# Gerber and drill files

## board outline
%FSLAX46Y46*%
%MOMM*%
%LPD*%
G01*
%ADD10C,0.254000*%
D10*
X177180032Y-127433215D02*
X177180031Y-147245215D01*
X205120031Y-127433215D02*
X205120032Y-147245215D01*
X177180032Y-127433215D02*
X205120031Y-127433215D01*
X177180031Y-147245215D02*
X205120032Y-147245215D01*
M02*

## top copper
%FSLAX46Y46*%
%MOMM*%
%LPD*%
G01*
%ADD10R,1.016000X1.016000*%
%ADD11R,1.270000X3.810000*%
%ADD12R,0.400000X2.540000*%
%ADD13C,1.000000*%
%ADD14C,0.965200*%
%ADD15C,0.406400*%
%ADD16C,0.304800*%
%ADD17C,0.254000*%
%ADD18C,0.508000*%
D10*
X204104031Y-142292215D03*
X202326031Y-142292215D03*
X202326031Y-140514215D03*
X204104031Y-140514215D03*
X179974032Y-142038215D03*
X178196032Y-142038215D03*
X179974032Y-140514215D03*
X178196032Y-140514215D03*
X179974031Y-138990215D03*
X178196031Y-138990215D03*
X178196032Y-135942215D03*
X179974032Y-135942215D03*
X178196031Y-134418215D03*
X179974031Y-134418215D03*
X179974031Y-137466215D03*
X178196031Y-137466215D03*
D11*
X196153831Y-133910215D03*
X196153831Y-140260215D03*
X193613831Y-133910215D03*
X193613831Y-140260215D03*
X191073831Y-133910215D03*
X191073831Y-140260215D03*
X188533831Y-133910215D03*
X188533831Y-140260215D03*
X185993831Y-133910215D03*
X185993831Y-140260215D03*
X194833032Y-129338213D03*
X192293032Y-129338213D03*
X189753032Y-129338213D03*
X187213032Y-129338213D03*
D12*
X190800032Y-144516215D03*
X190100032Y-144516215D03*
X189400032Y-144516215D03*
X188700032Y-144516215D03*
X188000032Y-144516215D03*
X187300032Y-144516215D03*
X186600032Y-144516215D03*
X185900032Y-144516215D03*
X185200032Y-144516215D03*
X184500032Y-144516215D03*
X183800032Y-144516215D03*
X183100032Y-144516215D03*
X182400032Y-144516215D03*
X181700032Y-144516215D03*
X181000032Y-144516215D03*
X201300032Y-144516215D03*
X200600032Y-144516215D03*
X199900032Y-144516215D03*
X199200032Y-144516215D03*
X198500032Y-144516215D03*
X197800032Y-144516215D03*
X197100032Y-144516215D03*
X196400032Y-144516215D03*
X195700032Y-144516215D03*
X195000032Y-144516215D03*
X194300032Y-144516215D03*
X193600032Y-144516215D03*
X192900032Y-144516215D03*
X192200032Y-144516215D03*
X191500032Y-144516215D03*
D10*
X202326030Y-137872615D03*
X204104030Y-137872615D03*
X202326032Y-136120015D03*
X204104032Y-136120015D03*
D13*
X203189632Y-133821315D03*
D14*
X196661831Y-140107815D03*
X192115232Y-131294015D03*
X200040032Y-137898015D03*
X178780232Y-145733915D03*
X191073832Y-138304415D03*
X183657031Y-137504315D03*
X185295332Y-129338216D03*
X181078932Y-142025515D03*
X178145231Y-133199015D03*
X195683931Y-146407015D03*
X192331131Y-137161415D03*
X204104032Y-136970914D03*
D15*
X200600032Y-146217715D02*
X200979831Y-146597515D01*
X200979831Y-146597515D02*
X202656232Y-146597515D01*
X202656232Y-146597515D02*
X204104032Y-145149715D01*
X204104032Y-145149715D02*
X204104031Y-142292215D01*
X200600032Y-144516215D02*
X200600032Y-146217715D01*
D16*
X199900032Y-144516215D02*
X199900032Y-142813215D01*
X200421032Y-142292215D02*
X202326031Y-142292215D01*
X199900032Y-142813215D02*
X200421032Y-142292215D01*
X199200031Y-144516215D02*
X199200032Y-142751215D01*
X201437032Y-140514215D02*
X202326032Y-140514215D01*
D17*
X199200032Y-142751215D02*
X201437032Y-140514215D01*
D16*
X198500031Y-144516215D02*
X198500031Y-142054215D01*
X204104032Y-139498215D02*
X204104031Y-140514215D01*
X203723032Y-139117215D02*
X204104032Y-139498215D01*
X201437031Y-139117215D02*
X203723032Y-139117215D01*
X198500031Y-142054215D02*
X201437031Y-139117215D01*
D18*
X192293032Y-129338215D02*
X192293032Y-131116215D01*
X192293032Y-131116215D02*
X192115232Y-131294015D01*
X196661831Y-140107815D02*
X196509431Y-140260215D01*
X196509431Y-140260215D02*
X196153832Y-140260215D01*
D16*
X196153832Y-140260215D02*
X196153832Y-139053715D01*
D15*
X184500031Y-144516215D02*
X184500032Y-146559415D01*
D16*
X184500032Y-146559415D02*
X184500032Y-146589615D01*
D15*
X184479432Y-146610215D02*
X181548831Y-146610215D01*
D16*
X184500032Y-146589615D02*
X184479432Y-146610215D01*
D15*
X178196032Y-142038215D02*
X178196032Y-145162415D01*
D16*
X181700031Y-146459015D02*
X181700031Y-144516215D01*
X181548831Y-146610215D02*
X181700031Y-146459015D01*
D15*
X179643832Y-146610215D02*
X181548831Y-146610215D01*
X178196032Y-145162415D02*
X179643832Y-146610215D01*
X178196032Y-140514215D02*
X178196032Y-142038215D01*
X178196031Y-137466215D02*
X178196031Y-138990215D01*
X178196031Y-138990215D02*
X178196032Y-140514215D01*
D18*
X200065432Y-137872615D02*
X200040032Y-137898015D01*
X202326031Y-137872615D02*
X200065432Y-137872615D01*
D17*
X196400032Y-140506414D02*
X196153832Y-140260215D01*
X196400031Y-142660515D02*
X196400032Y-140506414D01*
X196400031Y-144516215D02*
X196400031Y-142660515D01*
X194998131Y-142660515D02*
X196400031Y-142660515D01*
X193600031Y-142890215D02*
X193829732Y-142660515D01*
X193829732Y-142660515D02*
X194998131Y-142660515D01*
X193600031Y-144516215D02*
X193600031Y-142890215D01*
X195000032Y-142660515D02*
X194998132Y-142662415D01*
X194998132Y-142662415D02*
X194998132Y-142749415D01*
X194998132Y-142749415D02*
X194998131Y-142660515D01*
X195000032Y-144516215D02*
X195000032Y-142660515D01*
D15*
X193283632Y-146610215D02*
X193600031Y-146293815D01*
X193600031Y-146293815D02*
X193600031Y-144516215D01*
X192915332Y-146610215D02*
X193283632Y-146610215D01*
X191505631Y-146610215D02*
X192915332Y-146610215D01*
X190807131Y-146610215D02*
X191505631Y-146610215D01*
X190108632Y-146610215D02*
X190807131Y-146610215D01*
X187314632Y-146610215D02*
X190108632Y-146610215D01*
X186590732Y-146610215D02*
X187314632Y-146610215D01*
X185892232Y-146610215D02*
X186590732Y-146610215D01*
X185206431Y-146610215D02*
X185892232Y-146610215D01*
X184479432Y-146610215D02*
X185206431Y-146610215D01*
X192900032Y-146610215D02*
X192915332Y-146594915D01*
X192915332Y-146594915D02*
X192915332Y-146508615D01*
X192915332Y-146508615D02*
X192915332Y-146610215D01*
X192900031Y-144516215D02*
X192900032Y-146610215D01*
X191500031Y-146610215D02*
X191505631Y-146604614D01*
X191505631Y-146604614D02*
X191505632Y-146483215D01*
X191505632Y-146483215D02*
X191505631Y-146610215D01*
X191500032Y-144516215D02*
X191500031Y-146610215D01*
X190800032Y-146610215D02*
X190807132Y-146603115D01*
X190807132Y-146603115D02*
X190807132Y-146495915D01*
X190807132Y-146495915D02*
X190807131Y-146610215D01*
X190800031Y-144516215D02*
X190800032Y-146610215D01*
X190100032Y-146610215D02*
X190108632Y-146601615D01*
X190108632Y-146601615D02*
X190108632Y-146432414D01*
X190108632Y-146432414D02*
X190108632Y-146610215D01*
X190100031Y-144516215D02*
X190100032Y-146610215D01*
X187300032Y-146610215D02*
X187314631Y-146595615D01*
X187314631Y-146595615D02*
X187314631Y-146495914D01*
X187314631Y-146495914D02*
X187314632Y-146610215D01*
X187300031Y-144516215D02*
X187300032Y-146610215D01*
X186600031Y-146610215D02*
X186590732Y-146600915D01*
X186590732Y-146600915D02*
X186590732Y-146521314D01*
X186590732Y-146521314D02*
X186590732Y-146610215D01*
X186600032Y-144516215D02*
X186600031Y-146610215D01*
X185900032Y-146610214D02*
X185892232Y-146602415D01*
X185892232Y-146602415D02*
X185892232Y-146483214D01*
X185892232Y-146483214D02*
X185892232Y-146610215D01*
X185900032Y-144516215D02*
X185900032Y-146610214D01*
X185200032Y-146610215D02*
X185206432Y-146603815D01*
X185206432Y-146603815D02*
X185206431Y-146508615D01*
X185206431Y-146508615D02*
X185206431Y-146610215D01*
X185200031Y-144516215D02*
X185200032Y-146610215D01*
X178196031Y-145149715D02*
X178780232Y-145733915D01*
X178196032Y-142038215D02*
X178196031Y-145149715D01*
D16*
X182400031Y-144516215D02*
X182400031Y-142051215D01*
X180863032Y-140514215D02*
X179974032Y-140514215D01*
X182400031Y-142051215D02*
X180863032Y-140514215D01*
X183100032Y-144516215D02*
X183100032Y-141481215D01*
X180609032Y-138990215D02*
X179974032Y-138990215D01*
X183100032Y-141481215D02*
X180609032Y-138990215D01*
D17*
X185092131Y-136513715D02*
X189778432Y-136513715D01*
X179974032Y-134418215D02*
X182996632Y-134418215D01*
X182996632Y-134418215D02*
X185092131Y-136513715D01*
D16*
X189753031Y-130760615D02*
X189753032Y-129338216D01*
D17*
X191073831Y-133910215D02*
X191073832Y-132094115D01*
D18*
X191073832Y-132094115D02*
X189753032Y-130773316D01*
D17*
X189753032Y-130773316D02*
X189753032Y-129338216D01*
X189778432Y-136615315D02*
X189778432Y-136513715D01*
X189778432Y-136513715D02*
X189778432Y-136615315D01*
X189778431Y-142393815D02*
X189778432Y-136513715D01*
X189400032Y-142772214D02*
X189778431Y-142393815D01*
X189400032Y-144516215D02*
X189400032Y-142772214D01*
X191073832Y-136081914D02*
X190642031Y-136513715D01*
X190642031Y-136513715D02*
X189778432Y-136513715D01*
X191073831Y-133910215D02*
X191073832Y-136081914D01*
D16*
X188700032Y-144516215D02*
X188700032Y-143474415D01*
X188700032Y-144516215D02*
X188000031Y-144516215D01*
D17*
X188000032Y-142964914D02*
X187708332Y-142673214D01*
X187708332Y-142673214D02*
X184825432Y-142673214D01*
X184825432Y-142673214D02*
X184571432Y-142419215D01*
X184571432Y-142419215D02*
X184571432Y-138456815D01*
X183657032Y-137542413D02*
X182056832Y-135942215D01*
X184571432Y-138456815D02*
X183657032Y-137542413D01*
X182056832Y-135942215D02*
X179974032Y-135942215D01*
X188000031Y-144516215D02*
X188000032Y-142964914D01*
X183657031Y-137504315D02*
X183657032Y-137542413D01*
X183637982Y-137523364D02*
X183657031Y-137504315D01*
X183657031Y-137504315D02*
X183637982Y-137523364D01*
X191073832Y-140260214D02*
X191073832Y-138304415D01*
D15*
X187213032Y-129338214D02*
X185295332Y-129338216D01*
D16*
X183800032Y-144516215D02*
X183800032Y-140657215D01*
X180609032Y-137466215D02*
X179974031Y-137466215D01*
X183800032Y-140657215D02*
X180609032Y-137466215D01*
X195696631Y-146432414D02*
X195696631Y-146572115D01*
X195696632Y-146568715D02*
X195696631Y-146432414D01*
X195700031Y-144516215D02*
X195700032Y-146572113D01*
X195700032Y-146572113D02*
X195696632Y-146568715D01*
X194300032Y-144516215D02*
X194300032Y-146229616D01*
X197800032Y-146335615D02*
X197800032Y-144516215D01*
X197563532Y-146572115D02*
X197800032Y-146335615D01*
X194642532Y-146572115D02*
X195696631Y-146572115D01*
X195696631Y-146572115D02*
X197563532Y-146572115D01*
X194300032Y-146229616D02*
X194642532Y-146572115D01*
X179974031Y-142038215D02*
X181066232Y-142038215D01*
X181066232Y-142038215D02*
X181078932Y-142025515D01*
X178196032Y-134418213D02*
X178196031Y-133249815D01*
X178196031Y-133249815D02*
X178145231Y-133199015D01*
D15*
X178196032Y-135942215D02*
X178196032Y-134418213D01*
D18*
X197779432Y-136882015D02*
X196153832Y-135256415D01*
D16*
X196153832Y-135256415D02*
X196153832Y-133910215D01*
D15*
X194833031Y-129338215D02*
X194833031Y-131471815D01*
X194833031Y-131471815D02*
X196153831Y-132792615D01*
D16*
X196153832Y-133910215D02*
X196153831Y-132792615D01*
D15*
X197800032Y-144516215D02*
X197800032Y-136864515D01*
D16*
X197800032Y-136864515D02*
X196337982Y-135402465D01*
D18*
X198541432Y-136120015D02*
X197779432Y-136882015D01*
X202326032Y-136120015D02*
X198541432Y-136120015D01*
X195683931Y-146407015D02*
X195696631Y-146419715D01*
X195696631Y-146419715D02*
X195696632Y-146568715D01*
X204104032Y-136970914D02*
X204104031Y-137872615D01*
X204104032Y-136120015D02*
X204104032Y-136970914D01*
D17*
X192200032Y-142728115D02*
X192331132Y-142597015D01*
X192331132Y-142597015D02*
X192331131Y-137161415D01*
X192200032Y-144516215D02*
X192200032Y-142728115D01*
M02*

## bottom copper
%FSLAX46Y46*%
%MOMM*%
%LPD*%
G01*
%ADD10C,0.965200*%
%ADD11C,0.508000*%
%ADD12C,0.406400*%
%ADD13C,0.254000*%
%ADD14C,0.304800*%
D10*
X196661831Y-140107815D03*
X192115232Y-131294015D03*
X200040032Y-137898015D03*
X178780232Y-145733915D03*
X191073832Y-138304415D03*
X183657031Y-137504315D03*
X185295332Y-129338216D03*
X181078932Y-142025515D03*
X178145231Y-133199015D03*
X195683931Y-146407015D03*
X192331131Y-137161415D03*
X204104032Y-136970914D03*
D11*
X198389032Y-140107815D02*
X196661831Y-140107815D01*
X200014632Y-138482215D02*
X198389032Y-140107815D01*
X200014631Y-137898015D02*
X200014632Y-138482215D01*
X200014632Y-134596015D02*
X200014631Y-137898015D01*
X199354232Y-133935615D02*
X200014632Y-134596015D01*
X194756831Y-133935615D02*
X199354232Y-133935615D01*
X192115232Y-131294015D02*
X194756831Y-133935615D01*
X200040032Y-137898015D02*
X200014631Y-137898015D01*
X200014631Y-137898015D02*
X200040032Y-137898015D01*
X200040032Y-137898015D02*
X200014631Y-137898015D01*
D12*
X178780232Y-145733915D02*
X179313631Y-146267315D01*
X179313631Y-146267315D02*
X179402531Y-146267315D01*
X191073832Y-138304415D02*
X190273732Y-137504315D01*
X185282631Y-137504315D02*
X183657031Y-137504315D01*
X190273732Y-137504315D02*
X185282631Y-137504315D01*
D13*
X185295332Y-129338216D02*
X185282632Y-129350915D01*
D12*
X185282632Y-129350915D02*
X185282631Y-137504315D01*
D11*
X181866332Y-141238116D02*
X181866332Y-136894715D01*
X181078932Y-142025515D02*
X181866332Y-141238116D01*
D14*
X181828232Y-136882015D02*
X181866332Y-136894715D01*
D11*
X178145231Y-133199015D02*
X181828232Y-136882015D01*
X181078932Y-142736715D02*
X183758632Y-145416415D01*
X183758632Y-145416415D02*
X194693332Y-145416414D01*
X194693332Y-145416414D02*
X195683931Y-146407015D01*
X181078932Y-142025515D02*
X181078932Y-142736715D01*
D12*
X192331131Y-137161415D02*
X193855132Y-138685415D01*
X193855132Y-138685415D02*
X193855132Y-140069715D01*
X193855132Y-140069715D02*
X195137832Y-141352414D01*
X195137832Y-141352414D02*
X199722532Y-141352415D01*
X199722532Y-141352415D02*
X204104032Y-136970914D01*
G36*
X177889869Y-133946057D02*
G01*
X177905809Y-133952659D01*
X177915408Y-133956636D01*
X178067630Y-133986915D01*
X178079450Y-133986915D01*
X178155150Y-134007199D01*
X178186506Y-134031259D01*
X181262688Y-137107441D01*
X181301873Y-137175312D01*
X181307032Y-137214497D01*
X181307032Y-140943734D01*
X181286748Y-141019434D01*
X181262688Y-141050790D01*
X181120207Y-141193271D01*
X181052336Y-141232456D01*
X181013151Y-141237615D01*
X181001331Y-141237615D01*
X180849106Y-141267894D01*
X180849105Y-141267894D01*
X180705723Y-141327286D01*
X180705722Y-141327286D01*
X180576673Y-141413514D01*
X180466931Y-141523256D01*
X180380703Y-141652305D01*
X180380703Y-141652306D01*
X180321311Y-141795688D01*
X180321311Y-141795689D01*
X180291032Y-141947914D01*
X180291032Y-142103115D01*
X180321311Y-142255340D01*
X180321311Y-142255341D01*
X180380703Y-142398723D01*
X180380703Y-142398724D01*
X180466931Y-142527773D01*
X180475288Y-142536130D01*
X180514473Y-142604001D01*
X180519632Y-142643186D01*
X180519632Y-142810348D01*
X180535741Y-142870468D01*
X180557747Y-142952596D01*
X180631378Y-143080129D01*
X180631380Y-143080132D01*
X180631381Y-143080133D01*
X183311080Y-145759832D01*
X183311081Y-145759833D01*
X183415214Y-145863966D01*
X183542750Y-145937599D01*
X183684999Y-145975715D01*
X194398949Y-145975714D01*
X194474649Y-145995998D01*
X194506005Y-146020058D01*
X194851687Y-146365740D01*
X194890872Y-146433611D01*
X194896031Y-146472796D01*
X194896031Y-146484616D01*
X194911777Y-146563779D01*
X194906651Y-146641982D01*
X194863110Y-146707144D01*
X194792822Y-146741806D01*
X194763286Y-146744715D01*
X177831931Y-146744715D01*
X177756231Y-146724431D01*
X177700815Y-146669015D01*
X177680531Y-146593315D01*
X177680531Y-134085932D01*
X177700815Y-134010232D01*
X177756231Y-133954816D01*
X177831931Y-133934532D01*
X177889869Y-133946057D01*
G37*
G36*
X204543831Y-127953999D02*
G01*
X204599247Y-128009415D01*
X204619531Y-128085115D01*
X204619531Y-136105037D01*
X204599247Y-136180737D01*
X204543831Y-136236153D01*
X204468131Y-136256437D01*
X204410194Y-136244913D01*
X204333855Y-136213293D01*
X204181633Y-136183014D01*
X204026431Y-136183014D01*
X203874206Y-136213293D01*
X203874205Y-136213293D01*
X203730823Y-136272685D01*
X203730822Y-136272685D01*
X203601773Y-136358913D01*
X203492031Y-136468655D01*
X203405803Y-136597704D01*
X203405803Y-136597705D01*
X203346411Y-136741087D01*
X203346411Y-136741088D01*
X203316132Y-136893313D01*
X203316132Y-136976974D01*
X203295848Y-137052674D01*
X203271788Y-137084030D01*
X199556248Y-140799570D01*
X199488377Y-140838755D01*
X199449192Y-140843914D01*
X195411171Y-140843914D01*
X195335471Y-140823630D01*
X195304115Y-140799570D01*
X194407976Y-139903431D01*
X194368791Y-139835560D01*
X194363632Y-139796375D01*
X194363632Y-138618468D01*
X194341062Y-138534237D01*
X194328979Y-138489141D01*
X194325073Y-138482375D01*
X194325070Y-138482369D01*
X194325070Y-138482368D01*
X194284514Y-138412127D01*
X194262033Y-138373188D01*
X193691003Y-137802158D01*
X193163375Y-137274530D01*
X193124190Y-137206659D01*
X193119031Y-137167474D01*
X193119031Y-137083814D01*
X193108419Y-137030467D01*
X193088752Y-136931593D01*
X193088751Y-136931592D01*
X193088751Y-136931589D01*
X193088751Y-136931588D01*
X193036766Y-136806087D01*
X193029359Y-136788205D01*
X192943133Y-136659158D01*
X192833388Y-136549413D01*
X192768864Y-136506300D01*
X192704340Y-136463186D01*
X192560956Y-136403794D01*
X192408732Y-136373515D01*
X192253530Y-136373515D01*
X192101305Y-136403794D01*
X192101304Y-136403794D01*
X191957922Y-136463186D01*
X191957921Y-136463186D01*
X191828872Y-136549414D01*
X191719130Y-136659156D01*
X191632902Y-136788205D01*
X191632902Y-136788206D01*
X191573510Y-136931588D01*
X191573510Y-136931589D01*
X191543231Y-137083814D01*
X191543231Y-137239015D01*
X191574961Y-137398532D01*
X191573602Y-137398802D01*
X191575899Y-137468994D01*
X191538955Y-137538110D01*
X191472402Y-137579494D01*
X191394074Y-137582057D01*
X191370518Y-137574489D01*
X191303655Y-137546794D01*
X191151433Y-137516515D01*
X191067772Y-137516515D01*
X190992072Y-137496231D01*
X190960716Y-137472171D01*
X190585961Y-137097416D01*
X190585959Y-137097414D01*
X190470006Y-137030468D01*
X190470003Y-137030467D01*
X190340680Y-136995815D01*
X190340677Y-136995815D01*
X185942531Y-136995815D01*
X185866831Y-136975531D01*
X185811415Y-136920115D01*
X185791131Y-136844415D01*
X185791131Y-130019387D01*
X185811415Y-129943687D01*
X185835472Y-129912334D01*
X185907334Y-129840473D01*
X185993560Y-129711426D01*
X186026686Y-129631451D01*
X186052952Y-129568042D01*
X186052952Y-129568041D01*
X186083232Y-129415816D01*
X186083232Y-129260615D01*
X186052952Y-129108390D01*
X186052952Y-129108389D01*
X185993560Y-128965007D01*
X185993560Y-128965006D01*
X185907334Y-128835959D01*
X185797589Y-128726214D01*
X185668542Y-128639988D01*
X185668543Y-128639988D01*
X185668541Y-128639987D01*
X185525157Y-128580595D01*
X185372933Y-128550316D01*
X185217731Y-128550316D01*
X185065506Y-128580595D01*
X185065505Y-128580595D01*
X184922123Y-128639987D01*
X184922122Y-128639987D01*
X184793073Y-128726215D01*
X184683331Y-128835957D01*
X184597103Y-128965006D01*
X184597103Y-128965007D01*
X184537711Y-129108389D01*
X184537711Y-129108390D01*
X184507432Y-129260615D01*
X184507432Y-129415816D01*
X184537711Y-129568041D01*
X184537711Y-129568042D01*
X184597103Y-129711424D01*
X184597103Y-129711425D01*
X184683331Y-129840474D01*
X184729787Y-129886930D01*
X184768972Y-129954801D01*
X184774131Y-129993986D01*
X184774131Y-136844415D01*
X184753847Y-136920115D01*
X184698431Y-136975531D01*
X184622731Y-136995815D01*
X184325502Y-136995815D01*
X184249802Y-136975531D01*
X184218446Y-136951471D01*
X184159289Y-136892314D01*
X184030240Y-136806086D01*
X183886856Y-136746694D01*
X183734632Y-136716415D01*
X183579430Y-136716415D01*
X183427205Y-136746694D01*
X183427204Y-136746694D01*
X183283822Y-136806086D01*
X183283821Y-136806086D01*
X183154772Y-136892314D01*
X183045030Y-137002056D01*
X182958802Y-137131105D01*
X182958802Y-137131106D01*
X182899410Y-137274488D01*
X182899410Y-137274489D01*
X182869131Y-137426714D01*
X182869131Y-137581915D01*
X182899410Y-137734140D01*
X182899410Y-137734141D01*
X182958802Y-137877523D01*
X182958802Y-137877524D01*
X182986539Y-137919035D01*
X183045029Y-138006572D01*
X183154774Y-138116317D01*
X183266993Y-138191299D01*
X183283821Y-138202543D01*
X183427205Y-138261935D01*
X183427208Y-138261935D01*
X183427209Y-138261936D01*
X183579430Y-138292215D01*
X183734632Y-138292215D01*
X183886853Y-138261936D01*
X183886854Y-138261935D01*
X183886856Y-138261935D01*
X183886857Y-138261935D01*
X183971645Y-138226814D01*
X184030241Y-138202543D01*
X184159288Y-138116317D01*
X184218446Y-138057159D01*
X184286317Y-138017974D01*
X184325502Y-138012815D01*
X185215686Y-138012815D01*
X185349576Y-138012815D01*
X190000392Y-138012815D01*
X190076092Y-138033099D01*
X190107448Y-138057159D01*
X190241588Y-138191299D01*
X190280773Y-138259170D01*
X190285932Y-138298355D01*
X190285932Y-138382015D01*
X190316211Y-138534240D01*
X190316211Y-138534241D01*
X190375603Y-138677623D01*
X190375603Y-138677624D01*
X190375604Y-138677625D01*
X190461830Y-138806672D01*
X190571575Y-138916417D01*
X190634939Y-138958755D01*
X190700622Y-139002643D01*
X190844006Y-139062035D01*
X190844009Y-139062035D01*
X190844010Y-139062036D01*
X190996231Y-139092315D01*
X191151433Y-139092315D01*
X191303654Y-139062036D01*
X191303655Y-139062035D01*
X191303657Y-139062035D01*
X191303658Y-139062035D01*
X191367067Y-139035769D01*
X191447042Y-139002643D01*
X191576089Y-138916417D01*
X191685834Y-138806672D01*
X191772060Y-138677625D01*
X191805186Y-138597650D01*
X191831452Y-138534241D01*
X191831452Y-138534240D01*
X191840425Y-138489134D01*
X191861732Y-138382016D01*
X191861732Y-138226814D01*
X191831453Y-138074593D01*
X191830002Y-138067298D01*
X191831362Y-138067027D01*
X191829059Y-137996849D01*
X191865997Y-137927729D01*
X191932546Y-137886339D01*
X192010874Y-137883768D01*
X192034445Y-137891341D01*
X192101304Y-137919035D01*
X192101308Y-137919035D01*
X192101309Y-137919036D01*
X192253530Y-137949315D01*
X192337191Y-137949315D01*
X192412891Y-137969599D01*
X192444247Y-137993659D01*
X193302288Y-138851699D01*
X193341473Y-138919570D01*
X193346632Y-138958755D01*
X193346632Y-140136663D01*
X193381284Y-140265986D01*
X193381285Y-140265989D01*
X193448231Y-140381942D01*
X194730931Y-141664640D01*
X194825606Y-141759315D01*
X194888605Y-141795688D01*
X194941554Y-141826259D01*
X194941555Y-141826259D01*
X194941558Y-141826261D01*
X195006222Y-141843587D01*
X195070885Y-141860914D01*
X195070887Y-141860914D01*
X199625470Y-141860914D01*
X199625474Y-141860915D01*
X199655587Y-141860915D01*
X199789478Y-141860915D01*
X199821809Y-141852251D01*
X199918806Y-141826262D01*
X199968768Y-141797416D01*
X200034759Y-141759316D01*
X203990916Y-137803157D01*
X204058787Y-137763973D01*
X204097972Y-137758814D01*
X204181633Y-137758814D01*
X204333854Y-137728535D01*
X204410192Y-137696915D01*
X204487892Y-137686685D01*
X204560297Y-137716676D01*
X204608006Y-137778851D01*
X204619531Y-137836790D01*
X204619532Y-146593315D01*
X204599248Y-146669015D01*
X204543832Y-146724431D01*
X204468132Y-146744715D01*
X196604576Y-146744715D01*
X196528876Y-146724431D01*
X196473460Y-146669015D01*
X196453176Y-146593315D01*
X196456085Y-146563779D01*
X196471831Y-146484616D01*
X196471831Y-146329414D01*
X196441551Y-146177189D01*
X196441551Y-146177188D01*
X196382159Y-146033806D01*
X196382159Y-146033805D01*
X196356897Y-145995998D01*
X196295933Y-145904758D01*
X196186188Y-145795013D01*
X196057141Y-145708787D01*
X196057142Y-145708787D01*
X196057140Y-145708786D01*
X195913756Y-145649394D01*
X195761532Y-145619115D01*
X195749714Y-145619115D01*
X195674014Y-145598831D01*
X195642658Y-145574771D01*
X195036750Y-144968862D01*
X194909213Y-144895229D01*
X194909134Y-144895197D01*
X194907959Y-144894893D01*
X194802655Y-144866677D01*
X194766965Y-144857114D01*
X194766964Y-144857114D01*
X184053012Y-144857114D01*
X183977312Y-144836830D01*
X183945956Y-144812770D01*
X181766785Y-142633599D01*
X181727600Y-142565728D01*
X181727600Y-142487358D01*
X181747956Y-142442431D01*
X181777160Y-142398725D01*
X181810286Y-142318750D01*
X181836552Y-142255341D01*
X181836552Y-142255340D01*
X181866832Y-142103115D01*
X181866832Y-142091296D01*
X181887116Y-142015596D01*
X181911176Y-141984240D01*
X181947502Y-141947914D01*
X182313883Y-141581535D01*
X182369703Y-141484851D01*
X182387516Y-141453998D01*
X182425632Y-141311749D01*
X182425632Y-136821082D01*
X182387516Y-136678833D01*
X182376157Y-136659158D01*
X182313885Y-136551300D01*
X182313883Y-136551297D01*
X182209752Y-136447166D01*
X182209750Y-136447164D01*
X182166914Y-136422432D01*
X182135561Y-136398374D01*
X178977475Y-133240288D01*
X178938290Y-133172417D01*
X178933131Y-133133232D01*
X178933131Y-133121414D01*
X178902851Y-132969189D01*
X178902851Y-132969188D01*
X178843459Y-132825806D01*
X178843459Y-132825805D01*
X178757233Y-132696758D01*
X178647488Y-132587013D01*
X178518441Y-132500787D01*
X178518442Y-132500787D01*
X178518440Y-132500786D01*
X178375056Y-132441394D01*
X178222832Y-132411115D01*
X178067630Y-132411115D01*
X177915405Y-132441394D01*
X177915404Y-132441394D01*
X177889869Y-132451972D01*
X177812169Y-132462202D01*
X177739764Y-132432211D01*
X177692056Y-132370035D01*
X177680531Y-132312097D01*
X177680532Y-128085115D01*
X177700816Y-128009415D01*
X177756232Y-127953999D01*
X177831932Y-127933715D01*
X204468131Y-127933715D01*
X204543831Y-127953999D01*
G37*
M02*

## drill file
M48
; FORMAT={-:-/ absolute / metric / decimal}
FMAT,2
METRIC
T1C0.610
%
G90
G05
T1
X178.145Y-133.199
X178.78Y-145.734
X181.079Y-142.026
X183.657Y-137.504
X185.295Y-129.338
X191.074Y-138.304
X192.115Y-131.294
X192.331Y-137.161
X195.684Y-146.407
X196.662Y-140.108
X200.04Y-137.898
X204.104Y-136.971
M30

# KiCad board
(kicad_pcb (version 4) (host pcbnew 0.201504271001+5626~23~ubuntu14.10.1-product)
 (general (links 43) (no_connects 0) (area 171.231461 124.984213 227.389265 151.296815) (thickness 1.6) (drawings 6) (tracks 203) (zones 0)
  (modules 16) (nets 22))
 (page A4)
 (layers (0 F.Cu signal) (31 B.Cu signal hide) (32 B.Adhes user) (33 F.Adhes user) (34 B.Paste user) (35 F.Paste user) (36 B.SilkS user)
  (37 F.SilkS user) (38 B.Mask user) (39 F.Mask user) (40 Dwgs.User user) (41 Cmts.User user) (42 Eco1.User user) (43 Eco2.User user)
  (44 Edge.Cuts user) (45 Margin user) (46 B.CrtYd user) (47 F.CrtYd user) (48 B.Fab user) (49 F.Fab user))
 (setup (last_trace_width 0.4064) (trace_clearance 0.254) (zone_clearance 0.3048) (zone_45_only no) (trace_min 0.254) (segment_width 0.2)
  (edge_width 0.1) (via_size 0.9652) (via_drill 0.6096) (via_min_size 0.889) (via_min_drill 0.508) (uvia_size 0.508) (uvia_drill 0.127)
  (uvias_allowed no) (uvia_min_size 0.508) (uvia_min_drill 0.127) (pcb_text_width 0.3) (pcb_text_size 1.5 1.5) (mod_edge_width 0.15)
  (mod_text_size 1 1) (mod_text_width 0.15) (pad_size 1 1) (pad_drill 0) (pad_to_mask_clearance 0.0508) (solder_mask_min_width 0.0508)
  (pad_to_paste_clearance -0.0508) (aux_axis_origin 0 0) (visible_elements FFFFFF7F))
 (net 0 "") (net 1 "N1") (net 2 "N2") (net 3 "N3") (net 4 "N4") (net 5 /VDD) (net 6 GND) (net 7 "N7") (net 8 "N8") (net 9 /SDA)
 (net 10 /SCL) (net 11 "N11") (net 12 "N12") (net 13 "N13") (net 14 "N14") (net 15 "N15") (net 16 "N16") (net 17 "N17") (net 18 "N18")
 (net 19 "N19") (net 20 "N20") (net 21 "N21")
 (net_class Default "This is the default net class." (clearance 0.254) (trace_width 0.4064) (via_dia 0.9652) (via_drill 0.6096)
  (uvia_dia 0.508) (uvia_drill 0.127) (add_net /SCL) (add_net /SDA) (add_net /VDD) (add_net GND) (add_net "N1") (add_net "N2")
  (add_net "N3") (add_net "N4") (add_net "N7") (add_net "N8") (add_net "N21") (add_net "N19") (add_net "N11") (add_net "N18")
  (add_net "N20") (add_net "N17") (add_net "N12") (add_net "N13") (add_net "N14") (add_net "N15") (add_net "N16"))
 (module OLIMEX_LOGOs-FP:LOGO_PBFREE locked (layer F.Cu) (at 202.8444 130.2258)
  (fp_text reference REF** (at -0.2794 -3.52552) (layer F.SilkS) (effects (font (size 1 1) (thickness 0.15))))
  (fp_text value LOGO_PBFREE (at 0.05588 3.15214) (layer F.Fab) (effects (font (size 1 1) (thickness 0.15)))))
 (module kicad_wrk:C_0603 (layer F.Cu) (at 203.215031 142.292215 180)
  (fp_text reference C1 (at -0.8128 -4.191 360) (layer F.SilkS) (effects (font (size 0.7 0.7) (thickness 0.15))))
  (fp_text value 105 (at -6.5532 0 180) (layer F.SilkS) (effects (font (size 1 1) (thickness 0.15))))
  (pad 1 smd rect (at -0.889 0 180) (size 1.016 1.016) (layers F.Cu F.Paste F.Mask) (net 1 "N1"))
  (pad 2 smd rect (at 0.889 0 180) (size 1.016 1.016) (layers F.Cu F.Paste F.Mask) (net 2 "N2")))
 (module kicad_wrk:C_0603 (layer F.Cu) (at 203.215031 140.514215)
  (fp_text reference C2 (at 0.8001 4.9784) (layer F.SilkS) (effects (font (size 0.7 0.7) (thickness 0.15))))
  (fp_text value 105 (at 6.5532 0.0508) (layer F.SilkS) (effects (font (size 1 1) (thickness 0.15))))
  (pad 1 smd rect (at -0.889 0) (size 1.016 1.016) (layers F.Cu F.Paste F.Mask) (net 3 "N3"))
  (pad 2 smd rect (at 0.889 0) (size 1.016 1.016) (layers F.Cu F.Paste F.Mask) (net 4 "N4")))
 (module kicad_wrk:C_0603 (layer F.Cu) (at 179.085032 142.038215 180)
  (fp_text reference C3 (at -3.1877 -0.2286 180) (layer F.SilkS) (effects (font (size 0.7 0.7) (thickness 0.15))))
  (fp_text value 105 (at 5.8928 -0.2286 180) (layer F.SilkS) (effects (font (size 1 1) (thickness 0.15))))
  (pad 1 smd rect (at -0.889 0 180) (size 1.016 1.016) (layers F.Cu F.Paste F.Mask) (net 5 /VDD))
  (pad 2 smd rect (at 0.889 0 180) (size 1.016 1.016) (layers F.Cu F.Paste F.Mask) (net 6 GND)))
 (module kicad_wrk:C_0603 (layer F.Cu) (at 179.085032 140.514215 180)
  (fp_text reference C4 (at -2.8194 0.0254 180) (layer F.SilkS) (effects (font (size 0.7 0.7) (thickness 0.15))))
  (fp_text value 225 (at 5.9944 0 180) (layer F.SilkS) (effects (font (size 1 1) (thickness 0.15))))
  (pad 1 smd rect (at -0.889 0 180) (size 1.016 1.016) (layers F.Cu F.Paste F.Mask) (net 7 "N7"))
  (pad 2 smd rect (at 0.889 0 180) (size 1.016 1.016) (layers F.Cu F.Paste F.Mask) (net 6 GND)))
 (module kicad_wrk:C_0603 (layer F.Cu) (at 179.085031 138.990215 180)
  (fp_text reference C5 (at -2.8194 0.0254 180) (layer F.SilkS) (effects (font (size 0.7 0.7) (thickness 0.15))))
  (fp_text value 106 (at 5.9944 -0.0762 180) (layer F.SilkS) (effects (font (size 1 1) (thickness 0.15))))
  (pad 1 smd rect (at -0.889 0 180) (size 1.016 1.016) (layers F.Cu F.Paste F.Mask) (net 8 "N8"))
  (pad 2 smd rect (at 0.889 0 180) (size 1.016 1.016) (layers F.Cu F.Paste F.Mask) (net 6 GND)))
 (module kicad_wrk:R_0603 (layer F.Cu) (at 179.085032 135.942215)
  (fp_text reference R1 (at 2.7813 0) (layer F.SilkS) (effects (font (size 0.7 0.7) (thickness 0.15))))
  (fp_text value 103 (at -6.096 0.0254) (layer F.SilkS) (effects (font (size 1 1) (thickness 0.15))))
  (pad 1 smd rect (at -0.889 0) (size 1.016 1.016) (layers F.Cu F.Paste F.Mask) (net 5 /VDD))
  (pad 2 smd rect (at 0.889 0) (size 1.016 1.016) (layers F.Cu F.Paste F.Mask) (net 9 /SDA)))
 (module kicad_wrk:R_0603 (layer F.Cu) (at 179.085031 134.418215)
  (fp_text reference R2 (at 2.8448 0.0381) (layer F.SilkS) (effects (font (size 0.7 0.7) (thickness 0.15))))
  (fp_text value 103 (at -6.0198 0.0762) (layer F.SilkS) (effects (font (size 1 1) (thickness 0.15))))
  (pad 1 smd rect (at -0.889 0) (size 1.016 1.016) (layers F.Cu F.Paste F.Mask) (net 5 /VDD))
  (pad 2 smd rect (at 0.889 0) (size 1.016 1.016) (layers F.Cu F.Paste F.Mask) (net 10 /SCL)))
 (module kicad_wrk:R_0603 (layer F.Cu) (at 179.085031 137.466215 180)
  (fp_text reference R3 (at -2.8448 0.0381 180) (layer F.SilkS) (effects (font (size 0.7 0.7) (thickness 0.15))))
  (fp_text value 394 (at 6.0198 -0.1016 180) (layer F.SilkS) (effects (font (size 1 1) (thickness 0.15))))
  (pad 1 smd rect (at -0.889 0 180) (size 1.016 1.016) (layers F.Cu F.Paste F.Mask) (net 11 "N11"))
  (pad 2 smd rect (at 0.889 0 180) (size 1.016 1.016) (layers F.Cu F.Paste F.Mask) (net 6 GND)))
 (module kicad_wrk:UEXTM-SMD (layer F.Cu) (at 191.073831 137.085215)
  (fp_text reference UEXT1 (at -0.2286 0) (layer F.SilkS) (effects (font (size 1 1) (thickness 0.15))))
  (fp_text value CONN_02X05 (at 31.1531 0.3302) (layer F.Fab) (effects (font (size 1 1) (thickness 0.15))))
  (pad 1 smd rect (at 5.08 -3.175) (size 1.27 3.81) (layers F.Cu F.Paste F.Mask) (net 5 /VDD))
  (pad 2 smd rect (at 5.08 3.175) (size 1.27 3.81) (layers F.Cu F.Paste F.Mask) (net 6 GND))
  (pad 3 smd rect (at 2.54 -3.175) (size 1.27 3.81) (layers F.Cu F.Paste F.Mask) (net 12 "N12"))
  (pad 4 smd rect (at 2.54 3.175) (size 1.27 3.81) (layers F.Cu F.Paste F.Mask) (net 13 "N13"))
  (pad 5 smd rect (at 0 -3.175) (size 1.27 3.81) (layers F.Cu F.Paste F.Mask) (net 10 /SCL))
  (pad 6 smd rect (at 0 3.175) (size 1.27 3.81) (layers F.Cu F.Paste F.Mask) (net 9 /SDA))
  (pad 7 smd rect (at -2.54 -3.175) (size 1.27 3.81) (layers F.Cu F.Paste F.Mask) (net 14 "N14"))
  (pad 8 smd rect (at -2.54 3.175) (size 1.27 3.81) (layers F.Cu F.Paste F.Mask) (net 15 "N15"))
  (pad 9 smd rect (at -5.08 -3.175) (size 1.27 3.81) (layers F.Cu F.Paste F.Mask) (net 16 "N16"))
  (pad 10 smd rect (at -5.08 3.175) (size 1.27 3.81) (layers F.Cu F.Paste F.Mask) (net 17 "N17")))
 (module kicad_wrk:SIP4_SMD (layer F.Cu) (at 191.023032 129.338213 180)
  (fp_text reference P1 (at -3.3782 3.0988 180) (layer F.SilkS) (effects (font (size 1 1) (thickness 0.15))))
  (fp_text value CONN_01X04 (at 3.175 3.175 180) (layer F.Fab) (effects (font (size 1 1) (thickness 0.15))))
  (pad 1 smd rect (at -3.81 0 180) (size 1.27 3.81) (layers F.Cu F.Mask) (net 5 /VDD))
  (pad 2 smd rect (at -1.27 0 180) (size 1.27 3.81) (layers F.Cu F.Mask) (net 6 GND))
  (pad 3 smd rect (at 1.27 0 180) (size 1.27 3.81) (layers F.Cu F.Mask) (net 10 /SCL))
  (pad 4 smd rect (at 3.81 0 180) (size 1.27 3.81) (layers F.Cu F.Mask) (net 9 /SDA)))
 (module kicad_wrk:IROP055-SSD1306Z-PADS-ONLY (layer F.Cu) (at 191.150032 143.816215 180)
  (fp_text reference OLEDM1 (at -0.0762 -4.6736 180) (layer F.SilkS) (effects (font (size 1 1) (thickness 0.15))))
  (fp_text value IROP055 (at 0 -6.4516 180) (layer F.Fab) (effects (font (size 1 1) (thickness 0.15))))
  (pad 16 smd rect (at 0.35 -0.7 180) (size 0.4 2.54) (layers F.Cu F.Paste F.Mask) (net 6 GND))
  (pad 17 smd rect (at 1.05 -0.7 180) (size 0.4 2.54) (layers F.Cu F.Paste F.Mask) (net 6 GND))
  (pad 18 smd rect (at 1.75 -0.7 180) (size 0.4 2.54) (layers F.Cu F.Paste F.Mask) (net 10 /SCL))
  (pad 19 smd rect (at 2.45 -0.7 180) (size 0.4 2.54) (layers F.Cu F.Paste F.Mask) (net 9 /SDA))
  (pad 20 smd rect (at 3.15 -0.7 180) (size 0.4 2.54) (layers F.Cu F.Paste F.Mask) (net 9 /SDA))
  (pad 21 smd rect (at 3.85 -0.7 180) (size 0.4 2.54) (layers F.Cu F.Paste F.Mask) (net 6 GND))
  (pad 22 smd rect (at 4.55 -0.7 180) (size 0.4 2.54) (layers F.Cu F.Paste F.Mask) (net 6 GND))
  (pad 23 smd rect (at 5.25 -0.7 180) (size 0.4 2.54) (layers F.Cu F.Paste F.Mask) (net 6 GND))
  (pad 24 smd rect (at 5.95 -0.7 180) (size 0.4 2.54) (layers F.Cu F.Paste F.Mask) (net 6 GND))
  (pad 25 smd rect (at 6.65 -0.7 180) (size 0.4 2.54) (layers F.Cu F.Paste F.Mask) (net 6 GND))
  (pad 26 smd rect (at 7.35 -0.7 180) (size 0.4 2.54) (layers F.Cu F.Paste F.Mask) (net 11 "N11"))
  (pad 27 smd rect (at 8.05 -0.7 180) (size 0.4 2.54) (layers F.Cu F.Paste F.Mask) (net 8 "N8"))
  (pad 28 smd rect (at 8.75 -0.7 180) (size 0.4 2.54) (layers F.Cu F.Paste F.Mask) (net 7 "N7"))
  (pad 29 smd rect (at 9.45 -0.7 180) (size 0.4 2.54) (layers F.Cu F.Paste F.Mask) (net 6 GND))
  (pad 30 smd rect (at 10.15 -0.7 180) (size 0.4 2.54) (layers F.Cu F.Paste F.Mask) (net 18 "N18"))
  (pad 1 smd rect (at -10.15 -0.7 180) (size 0.4 2.54) (layers F.Cu F.Paste F.Mask) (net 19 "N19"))
  (pad 2 smd rect (at -9.45 -0.7 180) (size 0.4 2.54) (layers F.Cu F.Paste F.Mask) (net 1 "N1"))
  (pad 3 smd rect (at -8.75 -0.7 180) (size 0.4 2.54) (layers F.Cu F.Paste F.Mask) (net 2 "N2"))
  (pad 4 smd rect (at -8.05 -0.7 180) (size 0.4 2.54) (layers F.Cu F.Paste F.Mask) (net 3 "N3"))
  (pad 5 smd rect (at -7.35 -0.7 180) (size 0.4 2.54) (layers F.Cu F.Paste F.Mask) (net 4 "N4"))
  (pad 6 smd rect (at -6.65 -0.7 180) (size 0.4 2.54) (layers F.Cu F.Paste F.Mask) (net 5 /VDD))
  (pad 7 smd rect (at -5.95 -0.7 180) (size 0.4 2.54) (layers F.Cu F.Paste F.Mask) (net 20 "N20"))
  (pad 8 smd rect (at -5.25 -0.7 180) (size 0.4 2.54) (layers F.Cu F.Paste F.Mask) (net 6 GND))
  (pad 9 smd rect (at -4.55 -0.7 180) (size 0.4 2.54) (layers F.Cu F.Paste F.Mask) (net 5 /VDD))
  (pad 10 smd rect (at -3.85 -0.7 180) (size 0.4 2.54) (layers F.Cu F.Paste F.Mask) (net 6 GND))
  (pad 11 smd rect (at -3.15 -0.7 180) (size 0.4 2.54) (layers F.Cu F.Paste F.Mask) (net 5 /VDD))
  (pad 12 smd rect (at -2.45 -0.7 180) (size 0.4 2.54) (layers F.Cu F.Paste F.Mask) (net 6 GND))
  (pad 13 smd rect (at -1.75 -0.7 180) (size 0.4 2.54) (layers F.Cu F.Paste F.Mask) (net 6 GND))
  (pad 14 smd rect (at -1.05 -0.7 180) (size 0.4 2.54) (layers F.Cu F.Paste F.Mask) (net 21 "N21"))
  (pad 15 smd rect (at -0.35 -0.7 180) (size 0.4 2.54) (layers F.Cu F.Paste F.Mask) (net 6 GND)))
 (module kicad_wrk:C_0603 (layer F.Cu) (at 203.21503 137.872615)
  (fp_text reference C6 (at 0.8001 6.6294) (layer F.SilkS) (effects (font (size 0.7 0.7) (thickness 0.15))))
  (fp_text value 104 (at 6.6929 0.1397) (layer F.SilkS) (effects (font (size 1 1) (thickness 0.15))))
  (pad 1 smd rect (at -0.889 0) (size 1.016 1.016) (layers F.Cu F.Paste F.Mask) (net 6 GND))
  (pad 2 smd rect (at 0.889 0) (size 1.016 1.016) (layers F.Cu F.Paste F.Mask) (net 21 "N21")))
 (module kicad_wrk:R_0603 (layer F.Cu) (at 203.215032 136.120015)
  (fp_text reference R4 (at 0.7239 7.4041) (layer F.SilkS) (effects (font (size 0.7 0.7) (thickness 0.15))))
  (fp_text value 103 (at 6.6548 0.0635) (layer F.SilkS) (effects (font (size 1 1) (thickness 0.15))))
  (pad 1 smd rect (at -0.889 0) (size 1.016 1.016) (layers F.Cu F.Paste F.Mask) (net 5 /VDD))
  (pad 2 smd rect (at 0.889 0) (size 1.016 1.016) (layers F.Cu F.Paste F.Mask) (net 21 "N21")))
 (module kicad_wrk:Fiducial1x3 (layer F.Cu) (at 203.189632 133.821315 180)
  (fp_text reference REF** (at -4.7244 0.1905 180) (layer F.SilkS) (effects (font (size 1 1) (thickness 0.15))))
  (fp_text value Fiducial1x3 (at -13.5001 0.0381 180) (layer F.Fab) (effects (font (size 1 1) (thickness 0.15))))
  (pad Fid1 smd circle (at 0 0 180) (size 1 1) (layers F.Cu F.Mask)))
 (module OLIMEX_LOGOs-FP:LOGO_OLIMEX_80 (layer F.Cu) (at 180.837632 128.728615)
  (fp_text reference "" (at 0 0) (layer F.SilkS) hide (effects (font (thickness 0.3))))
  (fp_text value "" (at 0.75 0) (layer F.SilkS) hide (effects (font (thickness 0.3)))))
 (gr_line (start 177.180032 127.433215) (end 177.180031 147.245215) (angle 90) (layer Edge.Cuts) (width 0.254))
 (gr_line (start 205.120031 127.433215) (end 205.120032 147.245215) (angle 90) (layer Edge.Cuts) (width 0.254))
 (gr_line (start 177.180032 127.433215) (end 205.120031 127.433215) (angle 90) (layer Edge.Cuts) (width 0.254))
 (gr_line (start 177.180031 147.245215) (end 205.120032 147.245215) (angle 90) (layer Edge.Cuts) (width 0.254))
 (segment (start 200.600032 146.217715) (end 200.979831 146.597515) (width 0.4064) (layer F.Cu) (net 1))
 (segment (start 200.979831 146.597515) (end 202.656232 146.597515) (width 0.4064) (layer F.Cu) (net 1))
 (segment (start 202.656232 146.597515) (end 204.104032 145.149715) (width 0.4064) (layer F.Cu) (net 1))
 (segment (start 204.104032 145.149715) (end 204.104031 142.292215) (width 0.4064) (layer F.Cu) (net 1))
 (segment (start 200.600032 144.516215) (end 200.600032 146.217715) (width 0.4064) (layer F.Cu) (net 1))
 (segment (start 199.900032 144.516215) (end 199.900032 142.813215) (width 0.3048) (layer F.Cu) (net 2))
 (segment (start 200.421032 142.292215) (end 202.326031 142.292215) (width 0.3048) (layer F.Cu) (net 2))
 (segment (start 199.900032 142.813215) (end 200.421032 142.292215) (width 0.3048) (layer F.Cu) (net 2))
 (segment (start 199.200031 144.516215) (end 199.200032 142.751215) (width 0.3048) (layer F.Cu) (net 3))
 (segment (start 201.437032 140.514215) (end 202.326032 140.514215) (width 0.3048) (layer F.Cu) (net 3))
 (segment (start 199.200032 142.751215) (end 201.437032 140.514215) (width 0.254) (layer F.Cu) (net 3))
 (segment (start 198.500031 144.516215) (end 198.500031 142.054215) (width 0.3048) (layer F.Cu) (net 4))
 (segment (start 204.104032 139.498215) (end 204.104031 140.514215) (width 0.3048) (layer F.Cu) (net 4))
 (segment (start 203.723032 139.117215) (end 204.104032 139.498215) (width 0.3048) (layer F.Cu) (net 4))
 (segment (start 201.437031 139.117215) (end 203.723032 139.117215) (width 0.3048) (layer F.Cu) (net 4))
 (segment (start 198.500031 142.054215) (end 201.437031 139.117215) (width 0.3048) (layer F.Cu) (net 4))
 (segment (start 198.389032 140.107815) (end 196.661831 140.107815) (width 0.508) (layer B.Cu) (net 6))
 (segment (start 200.014632 138.482215) (end 198.389032 140.107815) (width 0.508) (layer B.Cu) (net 6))
 (segment (start 200.014631 137.898015) (end 200.014632 138.482215) (width 0.508) (layer B.Cu) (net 6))
 (segment (start 200.014632 134.596015) (end 200.014631 137.898015) (width 0.508) (layer B.Cu) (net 6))
 (segment (start 199.354232 133.935615) (end 200.014632 134.596015) (width 0.508) (layer B.Cu) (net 6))
 (segment (start 194.756831 133.935615) (end 199.354232 133.935615) (width 0.508) (layer B.Cu) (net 6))
 (segment (start 192.115232 131.294015) (end 194.756831 133.935615) (width 0.508) (layer B.Cu) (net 6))
 (segment (start 192.293032 129.338215) (end 192.293032 131.116215) (width 0.508) (layer F.Cu) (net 6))
 (segment (start 192.293032 131.116215) (end 192.115232 131.294015) (width 0.508) (layer F.Cu) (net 6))
 (segment (start 196.661831 140.107815) (end 196.509431 140.260215) (width 0.508) (layer F.Cu) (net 6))
 (via (at 196.661831 140.107815) (size 0.9652) (layers F.Cu B.Cu) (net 6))
 (via (at 192.115232 131.294015) (size 0.9652) (layers F.Cu B.Cu) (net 6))
 (segment (start 196.509431 140.260215) (end 196.153832 140.260215) (width 0.508) (layer F.Cu) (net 6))
 (segment (start 196.153832 140.260215) (end 196.153832 139.053715) (width 0.3048) (layer F.Cu) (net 6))
 (segment (start 184.500031 144.516215) (end 184.500032 146.559415) (width 0.4064) (layer F.Cu) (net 6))
 (segment (start 184.500032 146.559415) (end 184.500032 146.589615) (width 0.3048) (layer F.Cu) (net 6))
 (segment (start 184.479432 146.610215) (end 181.548831 146.610215) (width 0.4064) (layer F.Cu) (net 6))
 (segment (start 184.500032 146.589615) (end 184.479432 146.610215) (width 0.3048) (layer F.Cu) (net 6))
 (segment (start 178.196032 142.038215) (end 178.196032 145.162415) (width 0.4064) (layer F.Cu) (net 6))
 (segment (start 181.700031 146.459015) (end 181.700031 144.516215) (width 0.3048) (layer F.Cu) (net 6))
 (segment (start 181.548831 146.610215) (end 181.700031 146.459015) (width 0.3048) (layer F.Cu) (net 6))
 (segment (start 179.643832 146.610215) (end 181.548831 146.610215) (width 0.4064) (layer F.Cu) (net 6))
 (segment (start 178.196032 145.162415) (end 179.643832 146.610215) (width 0.4064) (layer F.Cu) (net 6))
 (segment (start 178.196032 140.514215) (end 178.196032 142.038215) (width 0.4064) (layer F.Cu) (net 6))
 (segment (start 178.196031 137.466215) (end 178.196031 138.990215) (width 0.4064) (layer F.Cu) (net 6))
 (segment (start 178.196031 138.990215) (end 178.196032 140.514215) (width 0.4064) (layer F.Cu) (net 6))
 (segment (start 200.040032 137.898015) (end 200.014631 137.898015) (width 0.508) (layer B.Cu) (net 6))
 (segment (start 200.014631 137.898015) (end 200.040032 137.898015) (width 0.508) (layer B.Cu) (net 6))
 (segment (start 200.040032 137.898015) (end 200.014631 137.898015) (width 0.508) (layer B.Cu) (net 6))
 (segment (start 200.065432 137.872615) (end 200.040032 137.898015) (width 0.508) (layer F.Cu) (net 6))
 (via (at 200.040032 137.898015) (size 0.9652) (layers F.Cu B.Cu) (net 6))
 (segment (start 202.326031 137.872615) (end 200.065432 137.872615) (width 0.508) (layer F.Cu) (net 6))
 (segment (start 196.400032 140.506414) (end 196.153832 140.260215) (width 0.254) (layer F.Cu) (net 6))
 (segment (start 196.400031 142.660515) (end 196.400032 140.506414) (width 0.254) (layer F.Cu) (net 6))
 (segment (start 196.400031 144.516215) (end 196.400031 142.660515) (width 0.254) (layer F.Cu) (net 6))
 (segment (start 194.998131 142.660515) (end 196.400031 142.660515) (width 0.254) (layer F.Cu) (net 6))
 (segment (start 193.600031 142.890215) (end 193.829732 142.660515) (width 0.254) (layer F.Cu) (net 6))
 (segment (start 193.829732 142.660515) (end 194.998131 142.660515) (width 0.254) (layer F.Cu) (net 6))
 (segment (start 193.600031 144.516215) (end 193.600031 142.890215) (width 0.254) (layer F.Cu) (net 6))
 (segment (start 195.000032 142.660515) (end 194.998132 142.662415) (width 0.254) (layer F.Cu) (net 6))
 (segment (start 194.998132 142.662415) (end 194.998132 142.749415) (width 0.254) (layer F.Cu) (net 6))
 (segment (start 194.998132 142.749415) (end 194.998131 142.660515) (width 0.254) (layer F.Cu) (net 6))
 (segment (start 195.000032 144.516215) (end 195.000032 142.660515) (width 0.254) (layer F.Cu) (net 6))
 (segment (start 193.283632 146.610215) (end 193.600031 146.293815) (width 0.4064) (layer F.Cu) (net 6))
 (segment (start 193.600031 146.293815) (end 193.600031 144.516215) (width 0.4064) (layer F.Cu) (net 6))
 (segment (start 192.915332 146.610215) (end 193.283632 146.610215) (width 0.4064) (layer F.Cu) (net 6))
 (segment (start 191.505631 146.610215) (end 192.915332 146.610215) (width 0.4064) (layer F.Cu) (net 6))
 (segment (start 190.807131 146.610215) (end 191.505631 146.610215) (width 0.4064) (layer F.Cu) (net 6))
 (segment (start 190.108632 146.610215) (end 190.807131 146.610215) (width 0.4064) (layer F.Cu) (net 6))
 (segment (start 187.314632 146.610215) (end 190.108632 146.610215) (width 0.4064) (layer F.Cu) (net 6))
 (segment (start 186.590732 146.610215) (end 187.314632 146.610215) (width 0.4064) (layer F.Cu) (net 6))
 (segment (start 185.892232 146.610215) (end 186.590732 146.610215) (width 0.4064) (layer F.Cu) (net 6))
 (segment (start 185.206431 146.610215) (end 185.892232 146.610215) (width 0.4064) (layer F.Cu) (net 6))
 (segment (start 184.479432 146.610215) (end 185.206431 146.610215) (width 0.4064) (layer F.Cu) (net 6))
 (segment (start 192.900032 146.610215) (end 192.915332 146.594915) (width 0.4064) (layer F.Cu) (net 6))
 (segment (start 192.915332 146.594915) (end 192.915332 146.508615) (width 0.4064) (layer F.Cu) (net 6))
 (segment (start 192.915332 146.508615) (end 192.915332 146.610215) (width 0.4064) (layer F.Cu) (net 6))
 (segment (start 192.900031 144.516215) (end 192.900032 146.610215) (width 0.4064) (layer F.Cu) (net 6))
 (segment (start 191.500031 146.610215) (end 191.505631 146.604614) (width 0.4064) (layer F.Cu) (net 6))
 (segment (start 191.505631 146.604614) (end 191.505632 146.483215) (width 0.4064) (layer F.Cu) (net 6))
 (segment (start 191.505632 146.483215) (end 191.505631 146.610215) (width 0.4064) (layer F.Cu) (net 6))
 (segment (start 191.500032 144.516215) (end 191.500031 146.610215) (width 0.4064) (layer F.Cu) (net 6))
 (segment (start 190.800032 146.610215) (end 190.807132 146.603115) (width 0.4064) (layer F.Cu) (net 6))
 (segment (start 190.807132 146.603115) (end 190.807132 146.495915) (width 0.4064) (layer F.Cu) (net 6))
 (segment (start 190.807132 146.495915) (end 190.807131 146.610215) (width 0.4064) (layer F.Cu) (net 6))
 (segment (start 190.800031 144.516215) (end 190.800032 146.610215) (width 0.4064) (layer F.Cu) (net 6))
 (segment (start 190.100032 146.610215) (end 190.108632 146.601615) (width 0.4064) (layer F.Cu) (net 6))
 (segment (start 190.108632 146.601615) (end 190.108632 146.432414) (width 0.4064) (layer F.Cu) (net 6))
 (segment (start 190.108632 146.432414) (end 190.108632 146.610215) (width 0.4064) (layer F.Cu) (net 6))
 (segment (start 190.100031 144.516215) (end 190.100032 146.610215) (width 0.4064) (layer F.Cu) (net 6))
 (segment (start 187.300032 146.610215) (end 187.314631 146.595615) (width 0.4064) (layer F.Cu) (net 6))
 (segment (start 187.314631 146.595615) (end 187.314631 146.495914) (width 0.4064) (layer F.Cu) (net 6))
 (segment (start 187.314631 146.495914) (end 187.314632 146.610215) (width 0.4064) (layer F.Cu) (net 6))
 (segment (start 187.300031 144.516215) (end 187.300032 146.610215) (width 0.4064) (layer F.Cu) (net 6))
 (segment (start 186.600031 146.610215) (end 186.590732 146.600915) (width 0.4064) (layer F.Cu) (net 6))
 (segment (start 186.590732 146.600915) (end 186.590732 146.521314) (width 0.4064) (layer F.Cu) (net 6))
 (segment (start 186.590732 146.521314) (end 186.590732 146.610215) (width 0.4064) (layer F.Cu) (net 6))
 (segment (start 186.600032 144.516215) (end 186.600031 146.610215) (width 0.4064) (layer F.Cu) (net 6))
 (segment (start 185.900032 146.610214) (end 185.892232 146.602415) (width 0.4064) (layer F.Cu) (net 6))
 (segment (start 185.892232 146.602415) (end 185.892232 146.483214) (width 0.4064) (layer F.Cu) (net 6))
 (segment (start 185.892232 146.483214) (end 185.892232 146.610215) (width 0.4064) (layer F.Cu) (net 6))
 (segment (start 185.900032 144.516215) (end 185.900032 146.610214) (width 0.4064) (layer F.Cu) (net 6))
 (segment (start 185.200032 146.610215) (end 185.206432 146.603815) (width 0.4064) (layer F.Cu) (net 6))
 (segment (start 185.206432 146.603815) (end 185.206431 146.508615) (width 0.4064) (layer F.Cu) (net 6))
 (segment (start 185.206431 146.508615) (end 185.206431 146.610215) (width 0.4064) (layer F.Cu) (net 6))
 (segment (start 185.200031 144.516215) (end 185.200032 146.610215) (width 0.4064) (layer F.Cu) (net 6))
 (segment (start 178.196031 145.149715) (end 178.780232 145.733915) (width 0.4064) (layer F.Cu) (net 6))
 (via (at 178.780232 145.733915) (size 0.9652) (layers F.Cu B.Cu) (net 6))
 (segment (start 178.780232 145.733915) (end 179.313631 146.267315) (width 0.4064) (layer B.Cu) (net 6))
 (segment (start 179.313631 146.267315) (end 179.402531 146.267315) (width 0.4064) (layer B.Cu) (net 6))
 (segment (start 178.196032 142.038215) (end 178.196031 145.149715) (width 0.4064) (layer F.Cu) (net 6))
 (segment (start 182.400031 144.516215) (end 182.400031 142.051215) (width 0.3048) (layer F.Cu) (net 7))
 (segment (start 180.863032 140.514215) (end 179.974032 140.514215) (width 0.3048) (layer F.Cu) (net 7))
 (segment (start 182.400031 142.051215) (end 180.863032 140.514215) (width 0.3048) (layer F.Cu) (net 7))
 (segment (start 183.100032 144.516215) (end 183.100032 141.481215) (width 0.3048) (layer F.Cu) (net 8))
 (segment (start 180.609032 138.990215) (end 179.974032 138.990215) (width 0.3048) (layer F.Cu) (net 8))
 (segment (start 183.100032 141.481215) (end 180.609032 138.990215) (width 0.3048) (layer F.Cu) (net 8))
 (segment (start 185.092131 136.513715) (end 189.778432 136.513715) (width 0.254) (layer F.Cu) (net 10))
 (segment (start 179.974032 134.418215) (end 182.996632 134.418215) (width 0.254) (layer F.Cu) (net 10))
 (segment (start 182.996632 134.418215) (end 185.092131 136.513715) (width 0.254) (layer F.Cu) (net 10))
 (segment (start 189.753031 130.760615) (end 189.753032 129.338216) (width 0.3048) (layer F.Cu) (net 10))
 (segment (start 191.073831 133.910215) (end 191.073832 132.094115) (width 0.254) (layer F.Cu) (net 10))
 (segment (start 191.073832 132.094115) (end 189.753032 130.773316) (width 0.508) (layer F.Cu) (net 10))
 (segment (start 189.753032 130.773316) (end 189.753032 129.338216) (width 0.254) (layer F.Cu) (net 10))
 (segment (start 189.778432 136.615315) (end 189.778432 136.513715) (width 0.254) (layer F.Cu) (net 10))
 (segment (start 189.778432 136.513715) (end 189.778432 136.615315) (width 0.254) (layer F.Cu) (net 10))
 (segment (start 189.778431 142.393815) (end 189.778432 136.513715) (width 0.254) (layer F.Cu) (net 10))
 (segment (start 189.400032 142.772214) (end 189.778431 142.393815) (width 0.254) (layer F.Cu) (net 10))
 (segment (start 189.400032 144.516215) (end 189.400032 142.772214) (width 0.254) (layer F.Cu) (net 10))
 (segment (start 191.073832 136.081914) (end 190.642031 136.513715) (width 0.254) (layer F.Cu) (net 10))
 (segment (start 190.642031 136.513715) (end 189.778432 136.513715) (width 0.254) (layer F.Cu) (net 10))
 (segment (start 191.073831 133.910215) (end 191.073832 136.081914) (width 0.254) (layer F.Cu) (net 10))
 (segment (start 188.700032 144.516215) (end 188.700032 143.474415) (width 0.3048) (layer F.Cu) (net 9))
 (segment (start 188.700032 144.516215) (end 188.000031 144.516215) (width 0.3048) (layer F.Cu) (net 9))
 (segment (start 188.000032 142.964914) (end 187.708332 142.673214) (width 0.254) (layer F.Cu) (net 9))
 (segment (start 187.708332 142.673214) (end 184.825432 142.673214) (width 0.254) (layer F.Cu) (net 9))
 (segment (start 184.825432 142.673214) (end 184.571432 142.419215) (width 0.254) (layer F.Cu) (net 9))
 (segment (start 184.571432 142.419215) (end 184.571432 138.456815) (width 0.254) (layer F.Cu) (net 9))
 (segment (start 183.657032 137.542413) (end 182.056832 135.942215) (width 0.254) (layer F.Cu) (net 9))
 (segment (start 184.571432 138.456815) (end 183.657032 137.542413) (width 0.254) (layer F.Cu) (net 9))
 (segment (start 182.056832 135.942215) (end 179.974032 135.942215) (width 0.254) (layer F.Cu) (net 9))
 (segment (start 188.000031 144.516215) (end 188.000032 142.964914) (width 0.254) (layer F.Cu) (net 9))
 (segment (start 183.657031 137.504315) (end 183.657032 137.542413) (width 0.254) (layer F.Cu) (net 9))
 (segment (start 183.637982 137.523364) (end 183.657031 137.504315) (width 0.254) (layer F.Cu) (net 9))
 (segment (start 183.657031 137.504315) (end 183.637982 137.523364) (width 0.254) (layer F.Cu) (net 9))
 (via (at 191.073832 138.304415) (size 0.9652) (layers F.Cu B.Cu) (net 9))
 (segment (start 191.073832 138.304415) (end 190.273732 137.504315) (width 0.4064) (layer B.Cu) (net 9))
 (segment (start 185.282631 137.504315) (end 183.657031 137.504315) (width 0.4064) (layer B.Cu) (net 9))
 (segment (start 190.273732 137.504315) (end 185.282631 137.504315) (width 0.4064) (layer B.Cu) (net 9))
 (via (at 183.657031 137.504315) (size 0.9652) (layers F.Cu B.Cu) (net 9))
 (segment (start 191.073832 140.260214) (end 191.073832 138.304415) (width 0.254) (layer F.Cu) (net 9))
 (via (at 185.295332 129.338216) (size 0.9652) (layers F.Cu B.Cu) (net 9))
 (segment (start 185.295332 129.338216) (end 185.282632 129.350915) (width 0.254) (layer B.Cu) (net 9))
 (segment (start 185.282632 129.350915) (end 185.282631 137.504315) (width 0.4064) (layer B.Cu) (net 9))
 (segment (start 187.213032 129.338214) (end 185.295332 129.338216) (width 0.4064) (layer F.Cu) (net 9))
 (segment (start 183.800032 144.516215) (end 183.800032 140.657215) (width 0.3048) (layer F.Cu) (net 11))
 (segment (start 180.609032 137.466215) (end 179.974031 137.466215) (width 0.3048) (layer F.Cu) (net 11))
 (segment (start 183.800032 140.657215) (end 180.609032 137.466215) (width 0.3048) (layer F.Cu) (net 11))
 (segment (start 181.866332 141.238116) (end 181.866332 136.894715) (width 0.508) (layer B.Cu) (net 5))
 (segment (start 181.078932 142.025515) (end 181.866332 141.238116) (width 0.508) (layer B.Cu) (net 5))
 (segment (start 181.828232 136.882015) (end 181.866332 136.894715) (width 0.3048) (layer B.Cu) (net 5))
 (segment (start 178.145231 133.199015) (end 181.828232 136.882015) (width 0.508) (layer B.Cu) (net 5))
 (segment (start 195.696631 146.432414) (end 195.696631 146.572115) (width 0.3048) (layer F.Cu) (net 5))
 (segment (start 195.696632 146.568715) (end 195.696631 146.432414) (width 0.3048) (layer F.Cu) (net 5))
 (segment (start 195.700031 144.516215) (end 195.700032 146.572113) (width 0.3048) (layer F.Cu) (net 5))
 (segment (start 195.700032 146.572113) (end 195.696632 146.568715) (width 0.3048) (layer F.Cu) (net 5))
 (segment (start 194.300032 144.516215) (end 194.300032 146.229616) (width 0.3048) (layer F.Cu) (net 5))
 (segment (start 197.800032 146.335615) (end 197.800032 144.516215) (width 0.3048) (layer F.Cu) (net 5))
 (segment (start 197.563532 146.572115) (end 197.800032 146.335615) (width 0.3048) (layer F.Cu) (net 5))
 (segment (start 194.642532 146.572115) (end 195.696631 146.572115) (width 0.3048) (layer F.Cu) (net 5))
 (segment (start 195.696631 146.572115) (end 197.563532 146.572115) (width 0.3048) (layer F.Cu) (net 5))
 (segment (start 194.300032 146.229616) (end 194.642532 146.572115) (width 0.3048) (layer F.Cu) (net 5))
 (segment (start 179.974031 142.038215) (end 181.066232 142.038215) (width 0.3048) (layer F.Cu) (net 5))
 (via (at 181.078932 142.025515) (size 0.9652) (layers F.Cu B.Cu) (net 5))
 (segment (start 181.066232 142.038215) (end 181.078932 142.025515) (width 0.3048) (layer F.Cu) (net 5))
 (segment (start 178.196032 134.418213) (end 178.196031 133.249815) (width 0.3048) (layer F.Cu) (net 5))
 (via (at 178.145231 133.199015) (size 0.9652) (layers F.Cu B.Cu) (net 5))
 (segment (start 178.196031 133.249815) (end 178.145231 133.199015) (width 0.3048) (layer F.Cu) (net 5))
 (segment (start 178.196032 135.942215) (end 178.196032 134.418213) (width 0.4064) (layer F.Cu) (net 5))
 (segment (start 197.779432 136.882015) (end 196.153832 135.256415) (width 0.508) (layer F.Cu) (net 5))
 (segment (start 196.153832 135.256415) (end 196.153832 133.910215) (width 0.3048) (layer F.Cu) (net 5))
 (segment (start 194.833031 129.338215) (end 194.833031 131.471815) (width 0.4064) (layer F.Cu) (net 5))
 (segment (start 194.833031 131.471815) (end 196.153831 132.792615) (width 0.4064) (layer F.Cu) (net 5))
 (segment (start 196.153832 133.910215) (end 196.153831 132.792615) (width 0.3048) (layer F.Cu) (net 5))
 (segment (start 197.800032 144.516215) (end 197.800032 136.864515) (width 0.4064) (layer F.Cu) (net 5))
 (segment (start 197.800032 136.864515) (end 196.337982 135.402465) (width 0.3048) (layer F.Cu) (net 5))
 (segment (start 198.541432 136.120015) (end 197.779432 136.882015) (width 0.508) (layer F.Cu) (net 5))
 (segment (start 202.326032 136.120015) (end 198.541432 136.120015) (width 0.508) (layer F.Cu) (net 5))
 (segment (start 181.078932 142.736715) (end 183.758632 145.416415) (width 0.508) (layer B.Cu) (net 5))
 (segment (start 183.758632 145.416415) (end 194.693332 145.416414) (width 0.508) (layer B.Cu) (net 5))
 (segment (start 194.693332 145.416414) (end 195.683931 146.407015) (width 0.508) (layer B.Cu) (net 5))
 (via (at 195.683931 146.407015) (size 0.9652) (layers F.Cu B.Cu) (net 5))
 (segment (start 195.683931 146.407015) (end 195.696631 146.419715) (width 0.508) (layer F.Cu) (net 5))
 (segment (start 195.696631 146.419715) (end 195.696632 146.568715) (width 0.508) (layer F.Cu) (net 5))
 (segment (start 181.078932 142.025515) (end 181.078932 142.736715) (width 0.508) (layer B.Cu) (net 5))
 (segment (start 204.104032 136.970914) (end 204.104031 137.872615) (width 0.508) (layer F.Cu) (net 21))
 (segment (start 204.104032 136.120015) (end 204.104032 136.970914) (width 0.508) (layer F.Cu) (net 21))
 (segment (start 192.200032 142.728115) (end 192.331132 142.597015) (width 0.254) (layer F.Cu) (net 21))
 (segment (start 192.331132 142.597015) (end 192.331131 137.161415) (width 0.254) (layer F.Cu) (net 21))
 (via (at 192.331131 137.161415) (size 0.9652) (layers F.Cu B.Cu) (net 21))
 (segment (start 192.331131 137.161415) (end 193.855132 138.685415) (width 0.4064) (layer B.Cu) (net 21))
 (segment (start 193.855132 138.685415) (end 193.855132 140.069715) (width 0.4064) (layer B.Cu) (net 21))
 (segment (start 193.855132 140.069715) (end 195.137832 141.352414) (width 0.4064) (layer B.Cu) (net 21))
 (segment (start 195.137832 141.352414) (end 199.722532 141.352415) (width 0.4064) (layer B.Cu) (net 21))
 (segment (start 199.722532 141.352415) (end 204.104032 136.970914) (width 0.4064) (layer B.Cu) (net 21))
 (via (at 204.104032 136.970914) (size 0.9652) (layers F.Cu B.Cu) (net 21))
 (segment (start 192.200032 144.516215) (end 192.200032 142.728115) (width 0.254) (layer F.Cu) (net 21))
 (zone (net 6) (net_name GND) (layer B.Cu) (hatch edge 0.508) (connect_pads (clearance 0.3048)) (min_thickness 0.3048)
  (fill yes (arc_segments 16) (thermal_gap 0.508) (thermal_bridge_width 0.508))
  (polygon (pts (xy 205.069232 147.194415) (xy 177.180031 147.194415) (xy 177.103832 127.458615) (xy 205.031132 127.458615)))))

